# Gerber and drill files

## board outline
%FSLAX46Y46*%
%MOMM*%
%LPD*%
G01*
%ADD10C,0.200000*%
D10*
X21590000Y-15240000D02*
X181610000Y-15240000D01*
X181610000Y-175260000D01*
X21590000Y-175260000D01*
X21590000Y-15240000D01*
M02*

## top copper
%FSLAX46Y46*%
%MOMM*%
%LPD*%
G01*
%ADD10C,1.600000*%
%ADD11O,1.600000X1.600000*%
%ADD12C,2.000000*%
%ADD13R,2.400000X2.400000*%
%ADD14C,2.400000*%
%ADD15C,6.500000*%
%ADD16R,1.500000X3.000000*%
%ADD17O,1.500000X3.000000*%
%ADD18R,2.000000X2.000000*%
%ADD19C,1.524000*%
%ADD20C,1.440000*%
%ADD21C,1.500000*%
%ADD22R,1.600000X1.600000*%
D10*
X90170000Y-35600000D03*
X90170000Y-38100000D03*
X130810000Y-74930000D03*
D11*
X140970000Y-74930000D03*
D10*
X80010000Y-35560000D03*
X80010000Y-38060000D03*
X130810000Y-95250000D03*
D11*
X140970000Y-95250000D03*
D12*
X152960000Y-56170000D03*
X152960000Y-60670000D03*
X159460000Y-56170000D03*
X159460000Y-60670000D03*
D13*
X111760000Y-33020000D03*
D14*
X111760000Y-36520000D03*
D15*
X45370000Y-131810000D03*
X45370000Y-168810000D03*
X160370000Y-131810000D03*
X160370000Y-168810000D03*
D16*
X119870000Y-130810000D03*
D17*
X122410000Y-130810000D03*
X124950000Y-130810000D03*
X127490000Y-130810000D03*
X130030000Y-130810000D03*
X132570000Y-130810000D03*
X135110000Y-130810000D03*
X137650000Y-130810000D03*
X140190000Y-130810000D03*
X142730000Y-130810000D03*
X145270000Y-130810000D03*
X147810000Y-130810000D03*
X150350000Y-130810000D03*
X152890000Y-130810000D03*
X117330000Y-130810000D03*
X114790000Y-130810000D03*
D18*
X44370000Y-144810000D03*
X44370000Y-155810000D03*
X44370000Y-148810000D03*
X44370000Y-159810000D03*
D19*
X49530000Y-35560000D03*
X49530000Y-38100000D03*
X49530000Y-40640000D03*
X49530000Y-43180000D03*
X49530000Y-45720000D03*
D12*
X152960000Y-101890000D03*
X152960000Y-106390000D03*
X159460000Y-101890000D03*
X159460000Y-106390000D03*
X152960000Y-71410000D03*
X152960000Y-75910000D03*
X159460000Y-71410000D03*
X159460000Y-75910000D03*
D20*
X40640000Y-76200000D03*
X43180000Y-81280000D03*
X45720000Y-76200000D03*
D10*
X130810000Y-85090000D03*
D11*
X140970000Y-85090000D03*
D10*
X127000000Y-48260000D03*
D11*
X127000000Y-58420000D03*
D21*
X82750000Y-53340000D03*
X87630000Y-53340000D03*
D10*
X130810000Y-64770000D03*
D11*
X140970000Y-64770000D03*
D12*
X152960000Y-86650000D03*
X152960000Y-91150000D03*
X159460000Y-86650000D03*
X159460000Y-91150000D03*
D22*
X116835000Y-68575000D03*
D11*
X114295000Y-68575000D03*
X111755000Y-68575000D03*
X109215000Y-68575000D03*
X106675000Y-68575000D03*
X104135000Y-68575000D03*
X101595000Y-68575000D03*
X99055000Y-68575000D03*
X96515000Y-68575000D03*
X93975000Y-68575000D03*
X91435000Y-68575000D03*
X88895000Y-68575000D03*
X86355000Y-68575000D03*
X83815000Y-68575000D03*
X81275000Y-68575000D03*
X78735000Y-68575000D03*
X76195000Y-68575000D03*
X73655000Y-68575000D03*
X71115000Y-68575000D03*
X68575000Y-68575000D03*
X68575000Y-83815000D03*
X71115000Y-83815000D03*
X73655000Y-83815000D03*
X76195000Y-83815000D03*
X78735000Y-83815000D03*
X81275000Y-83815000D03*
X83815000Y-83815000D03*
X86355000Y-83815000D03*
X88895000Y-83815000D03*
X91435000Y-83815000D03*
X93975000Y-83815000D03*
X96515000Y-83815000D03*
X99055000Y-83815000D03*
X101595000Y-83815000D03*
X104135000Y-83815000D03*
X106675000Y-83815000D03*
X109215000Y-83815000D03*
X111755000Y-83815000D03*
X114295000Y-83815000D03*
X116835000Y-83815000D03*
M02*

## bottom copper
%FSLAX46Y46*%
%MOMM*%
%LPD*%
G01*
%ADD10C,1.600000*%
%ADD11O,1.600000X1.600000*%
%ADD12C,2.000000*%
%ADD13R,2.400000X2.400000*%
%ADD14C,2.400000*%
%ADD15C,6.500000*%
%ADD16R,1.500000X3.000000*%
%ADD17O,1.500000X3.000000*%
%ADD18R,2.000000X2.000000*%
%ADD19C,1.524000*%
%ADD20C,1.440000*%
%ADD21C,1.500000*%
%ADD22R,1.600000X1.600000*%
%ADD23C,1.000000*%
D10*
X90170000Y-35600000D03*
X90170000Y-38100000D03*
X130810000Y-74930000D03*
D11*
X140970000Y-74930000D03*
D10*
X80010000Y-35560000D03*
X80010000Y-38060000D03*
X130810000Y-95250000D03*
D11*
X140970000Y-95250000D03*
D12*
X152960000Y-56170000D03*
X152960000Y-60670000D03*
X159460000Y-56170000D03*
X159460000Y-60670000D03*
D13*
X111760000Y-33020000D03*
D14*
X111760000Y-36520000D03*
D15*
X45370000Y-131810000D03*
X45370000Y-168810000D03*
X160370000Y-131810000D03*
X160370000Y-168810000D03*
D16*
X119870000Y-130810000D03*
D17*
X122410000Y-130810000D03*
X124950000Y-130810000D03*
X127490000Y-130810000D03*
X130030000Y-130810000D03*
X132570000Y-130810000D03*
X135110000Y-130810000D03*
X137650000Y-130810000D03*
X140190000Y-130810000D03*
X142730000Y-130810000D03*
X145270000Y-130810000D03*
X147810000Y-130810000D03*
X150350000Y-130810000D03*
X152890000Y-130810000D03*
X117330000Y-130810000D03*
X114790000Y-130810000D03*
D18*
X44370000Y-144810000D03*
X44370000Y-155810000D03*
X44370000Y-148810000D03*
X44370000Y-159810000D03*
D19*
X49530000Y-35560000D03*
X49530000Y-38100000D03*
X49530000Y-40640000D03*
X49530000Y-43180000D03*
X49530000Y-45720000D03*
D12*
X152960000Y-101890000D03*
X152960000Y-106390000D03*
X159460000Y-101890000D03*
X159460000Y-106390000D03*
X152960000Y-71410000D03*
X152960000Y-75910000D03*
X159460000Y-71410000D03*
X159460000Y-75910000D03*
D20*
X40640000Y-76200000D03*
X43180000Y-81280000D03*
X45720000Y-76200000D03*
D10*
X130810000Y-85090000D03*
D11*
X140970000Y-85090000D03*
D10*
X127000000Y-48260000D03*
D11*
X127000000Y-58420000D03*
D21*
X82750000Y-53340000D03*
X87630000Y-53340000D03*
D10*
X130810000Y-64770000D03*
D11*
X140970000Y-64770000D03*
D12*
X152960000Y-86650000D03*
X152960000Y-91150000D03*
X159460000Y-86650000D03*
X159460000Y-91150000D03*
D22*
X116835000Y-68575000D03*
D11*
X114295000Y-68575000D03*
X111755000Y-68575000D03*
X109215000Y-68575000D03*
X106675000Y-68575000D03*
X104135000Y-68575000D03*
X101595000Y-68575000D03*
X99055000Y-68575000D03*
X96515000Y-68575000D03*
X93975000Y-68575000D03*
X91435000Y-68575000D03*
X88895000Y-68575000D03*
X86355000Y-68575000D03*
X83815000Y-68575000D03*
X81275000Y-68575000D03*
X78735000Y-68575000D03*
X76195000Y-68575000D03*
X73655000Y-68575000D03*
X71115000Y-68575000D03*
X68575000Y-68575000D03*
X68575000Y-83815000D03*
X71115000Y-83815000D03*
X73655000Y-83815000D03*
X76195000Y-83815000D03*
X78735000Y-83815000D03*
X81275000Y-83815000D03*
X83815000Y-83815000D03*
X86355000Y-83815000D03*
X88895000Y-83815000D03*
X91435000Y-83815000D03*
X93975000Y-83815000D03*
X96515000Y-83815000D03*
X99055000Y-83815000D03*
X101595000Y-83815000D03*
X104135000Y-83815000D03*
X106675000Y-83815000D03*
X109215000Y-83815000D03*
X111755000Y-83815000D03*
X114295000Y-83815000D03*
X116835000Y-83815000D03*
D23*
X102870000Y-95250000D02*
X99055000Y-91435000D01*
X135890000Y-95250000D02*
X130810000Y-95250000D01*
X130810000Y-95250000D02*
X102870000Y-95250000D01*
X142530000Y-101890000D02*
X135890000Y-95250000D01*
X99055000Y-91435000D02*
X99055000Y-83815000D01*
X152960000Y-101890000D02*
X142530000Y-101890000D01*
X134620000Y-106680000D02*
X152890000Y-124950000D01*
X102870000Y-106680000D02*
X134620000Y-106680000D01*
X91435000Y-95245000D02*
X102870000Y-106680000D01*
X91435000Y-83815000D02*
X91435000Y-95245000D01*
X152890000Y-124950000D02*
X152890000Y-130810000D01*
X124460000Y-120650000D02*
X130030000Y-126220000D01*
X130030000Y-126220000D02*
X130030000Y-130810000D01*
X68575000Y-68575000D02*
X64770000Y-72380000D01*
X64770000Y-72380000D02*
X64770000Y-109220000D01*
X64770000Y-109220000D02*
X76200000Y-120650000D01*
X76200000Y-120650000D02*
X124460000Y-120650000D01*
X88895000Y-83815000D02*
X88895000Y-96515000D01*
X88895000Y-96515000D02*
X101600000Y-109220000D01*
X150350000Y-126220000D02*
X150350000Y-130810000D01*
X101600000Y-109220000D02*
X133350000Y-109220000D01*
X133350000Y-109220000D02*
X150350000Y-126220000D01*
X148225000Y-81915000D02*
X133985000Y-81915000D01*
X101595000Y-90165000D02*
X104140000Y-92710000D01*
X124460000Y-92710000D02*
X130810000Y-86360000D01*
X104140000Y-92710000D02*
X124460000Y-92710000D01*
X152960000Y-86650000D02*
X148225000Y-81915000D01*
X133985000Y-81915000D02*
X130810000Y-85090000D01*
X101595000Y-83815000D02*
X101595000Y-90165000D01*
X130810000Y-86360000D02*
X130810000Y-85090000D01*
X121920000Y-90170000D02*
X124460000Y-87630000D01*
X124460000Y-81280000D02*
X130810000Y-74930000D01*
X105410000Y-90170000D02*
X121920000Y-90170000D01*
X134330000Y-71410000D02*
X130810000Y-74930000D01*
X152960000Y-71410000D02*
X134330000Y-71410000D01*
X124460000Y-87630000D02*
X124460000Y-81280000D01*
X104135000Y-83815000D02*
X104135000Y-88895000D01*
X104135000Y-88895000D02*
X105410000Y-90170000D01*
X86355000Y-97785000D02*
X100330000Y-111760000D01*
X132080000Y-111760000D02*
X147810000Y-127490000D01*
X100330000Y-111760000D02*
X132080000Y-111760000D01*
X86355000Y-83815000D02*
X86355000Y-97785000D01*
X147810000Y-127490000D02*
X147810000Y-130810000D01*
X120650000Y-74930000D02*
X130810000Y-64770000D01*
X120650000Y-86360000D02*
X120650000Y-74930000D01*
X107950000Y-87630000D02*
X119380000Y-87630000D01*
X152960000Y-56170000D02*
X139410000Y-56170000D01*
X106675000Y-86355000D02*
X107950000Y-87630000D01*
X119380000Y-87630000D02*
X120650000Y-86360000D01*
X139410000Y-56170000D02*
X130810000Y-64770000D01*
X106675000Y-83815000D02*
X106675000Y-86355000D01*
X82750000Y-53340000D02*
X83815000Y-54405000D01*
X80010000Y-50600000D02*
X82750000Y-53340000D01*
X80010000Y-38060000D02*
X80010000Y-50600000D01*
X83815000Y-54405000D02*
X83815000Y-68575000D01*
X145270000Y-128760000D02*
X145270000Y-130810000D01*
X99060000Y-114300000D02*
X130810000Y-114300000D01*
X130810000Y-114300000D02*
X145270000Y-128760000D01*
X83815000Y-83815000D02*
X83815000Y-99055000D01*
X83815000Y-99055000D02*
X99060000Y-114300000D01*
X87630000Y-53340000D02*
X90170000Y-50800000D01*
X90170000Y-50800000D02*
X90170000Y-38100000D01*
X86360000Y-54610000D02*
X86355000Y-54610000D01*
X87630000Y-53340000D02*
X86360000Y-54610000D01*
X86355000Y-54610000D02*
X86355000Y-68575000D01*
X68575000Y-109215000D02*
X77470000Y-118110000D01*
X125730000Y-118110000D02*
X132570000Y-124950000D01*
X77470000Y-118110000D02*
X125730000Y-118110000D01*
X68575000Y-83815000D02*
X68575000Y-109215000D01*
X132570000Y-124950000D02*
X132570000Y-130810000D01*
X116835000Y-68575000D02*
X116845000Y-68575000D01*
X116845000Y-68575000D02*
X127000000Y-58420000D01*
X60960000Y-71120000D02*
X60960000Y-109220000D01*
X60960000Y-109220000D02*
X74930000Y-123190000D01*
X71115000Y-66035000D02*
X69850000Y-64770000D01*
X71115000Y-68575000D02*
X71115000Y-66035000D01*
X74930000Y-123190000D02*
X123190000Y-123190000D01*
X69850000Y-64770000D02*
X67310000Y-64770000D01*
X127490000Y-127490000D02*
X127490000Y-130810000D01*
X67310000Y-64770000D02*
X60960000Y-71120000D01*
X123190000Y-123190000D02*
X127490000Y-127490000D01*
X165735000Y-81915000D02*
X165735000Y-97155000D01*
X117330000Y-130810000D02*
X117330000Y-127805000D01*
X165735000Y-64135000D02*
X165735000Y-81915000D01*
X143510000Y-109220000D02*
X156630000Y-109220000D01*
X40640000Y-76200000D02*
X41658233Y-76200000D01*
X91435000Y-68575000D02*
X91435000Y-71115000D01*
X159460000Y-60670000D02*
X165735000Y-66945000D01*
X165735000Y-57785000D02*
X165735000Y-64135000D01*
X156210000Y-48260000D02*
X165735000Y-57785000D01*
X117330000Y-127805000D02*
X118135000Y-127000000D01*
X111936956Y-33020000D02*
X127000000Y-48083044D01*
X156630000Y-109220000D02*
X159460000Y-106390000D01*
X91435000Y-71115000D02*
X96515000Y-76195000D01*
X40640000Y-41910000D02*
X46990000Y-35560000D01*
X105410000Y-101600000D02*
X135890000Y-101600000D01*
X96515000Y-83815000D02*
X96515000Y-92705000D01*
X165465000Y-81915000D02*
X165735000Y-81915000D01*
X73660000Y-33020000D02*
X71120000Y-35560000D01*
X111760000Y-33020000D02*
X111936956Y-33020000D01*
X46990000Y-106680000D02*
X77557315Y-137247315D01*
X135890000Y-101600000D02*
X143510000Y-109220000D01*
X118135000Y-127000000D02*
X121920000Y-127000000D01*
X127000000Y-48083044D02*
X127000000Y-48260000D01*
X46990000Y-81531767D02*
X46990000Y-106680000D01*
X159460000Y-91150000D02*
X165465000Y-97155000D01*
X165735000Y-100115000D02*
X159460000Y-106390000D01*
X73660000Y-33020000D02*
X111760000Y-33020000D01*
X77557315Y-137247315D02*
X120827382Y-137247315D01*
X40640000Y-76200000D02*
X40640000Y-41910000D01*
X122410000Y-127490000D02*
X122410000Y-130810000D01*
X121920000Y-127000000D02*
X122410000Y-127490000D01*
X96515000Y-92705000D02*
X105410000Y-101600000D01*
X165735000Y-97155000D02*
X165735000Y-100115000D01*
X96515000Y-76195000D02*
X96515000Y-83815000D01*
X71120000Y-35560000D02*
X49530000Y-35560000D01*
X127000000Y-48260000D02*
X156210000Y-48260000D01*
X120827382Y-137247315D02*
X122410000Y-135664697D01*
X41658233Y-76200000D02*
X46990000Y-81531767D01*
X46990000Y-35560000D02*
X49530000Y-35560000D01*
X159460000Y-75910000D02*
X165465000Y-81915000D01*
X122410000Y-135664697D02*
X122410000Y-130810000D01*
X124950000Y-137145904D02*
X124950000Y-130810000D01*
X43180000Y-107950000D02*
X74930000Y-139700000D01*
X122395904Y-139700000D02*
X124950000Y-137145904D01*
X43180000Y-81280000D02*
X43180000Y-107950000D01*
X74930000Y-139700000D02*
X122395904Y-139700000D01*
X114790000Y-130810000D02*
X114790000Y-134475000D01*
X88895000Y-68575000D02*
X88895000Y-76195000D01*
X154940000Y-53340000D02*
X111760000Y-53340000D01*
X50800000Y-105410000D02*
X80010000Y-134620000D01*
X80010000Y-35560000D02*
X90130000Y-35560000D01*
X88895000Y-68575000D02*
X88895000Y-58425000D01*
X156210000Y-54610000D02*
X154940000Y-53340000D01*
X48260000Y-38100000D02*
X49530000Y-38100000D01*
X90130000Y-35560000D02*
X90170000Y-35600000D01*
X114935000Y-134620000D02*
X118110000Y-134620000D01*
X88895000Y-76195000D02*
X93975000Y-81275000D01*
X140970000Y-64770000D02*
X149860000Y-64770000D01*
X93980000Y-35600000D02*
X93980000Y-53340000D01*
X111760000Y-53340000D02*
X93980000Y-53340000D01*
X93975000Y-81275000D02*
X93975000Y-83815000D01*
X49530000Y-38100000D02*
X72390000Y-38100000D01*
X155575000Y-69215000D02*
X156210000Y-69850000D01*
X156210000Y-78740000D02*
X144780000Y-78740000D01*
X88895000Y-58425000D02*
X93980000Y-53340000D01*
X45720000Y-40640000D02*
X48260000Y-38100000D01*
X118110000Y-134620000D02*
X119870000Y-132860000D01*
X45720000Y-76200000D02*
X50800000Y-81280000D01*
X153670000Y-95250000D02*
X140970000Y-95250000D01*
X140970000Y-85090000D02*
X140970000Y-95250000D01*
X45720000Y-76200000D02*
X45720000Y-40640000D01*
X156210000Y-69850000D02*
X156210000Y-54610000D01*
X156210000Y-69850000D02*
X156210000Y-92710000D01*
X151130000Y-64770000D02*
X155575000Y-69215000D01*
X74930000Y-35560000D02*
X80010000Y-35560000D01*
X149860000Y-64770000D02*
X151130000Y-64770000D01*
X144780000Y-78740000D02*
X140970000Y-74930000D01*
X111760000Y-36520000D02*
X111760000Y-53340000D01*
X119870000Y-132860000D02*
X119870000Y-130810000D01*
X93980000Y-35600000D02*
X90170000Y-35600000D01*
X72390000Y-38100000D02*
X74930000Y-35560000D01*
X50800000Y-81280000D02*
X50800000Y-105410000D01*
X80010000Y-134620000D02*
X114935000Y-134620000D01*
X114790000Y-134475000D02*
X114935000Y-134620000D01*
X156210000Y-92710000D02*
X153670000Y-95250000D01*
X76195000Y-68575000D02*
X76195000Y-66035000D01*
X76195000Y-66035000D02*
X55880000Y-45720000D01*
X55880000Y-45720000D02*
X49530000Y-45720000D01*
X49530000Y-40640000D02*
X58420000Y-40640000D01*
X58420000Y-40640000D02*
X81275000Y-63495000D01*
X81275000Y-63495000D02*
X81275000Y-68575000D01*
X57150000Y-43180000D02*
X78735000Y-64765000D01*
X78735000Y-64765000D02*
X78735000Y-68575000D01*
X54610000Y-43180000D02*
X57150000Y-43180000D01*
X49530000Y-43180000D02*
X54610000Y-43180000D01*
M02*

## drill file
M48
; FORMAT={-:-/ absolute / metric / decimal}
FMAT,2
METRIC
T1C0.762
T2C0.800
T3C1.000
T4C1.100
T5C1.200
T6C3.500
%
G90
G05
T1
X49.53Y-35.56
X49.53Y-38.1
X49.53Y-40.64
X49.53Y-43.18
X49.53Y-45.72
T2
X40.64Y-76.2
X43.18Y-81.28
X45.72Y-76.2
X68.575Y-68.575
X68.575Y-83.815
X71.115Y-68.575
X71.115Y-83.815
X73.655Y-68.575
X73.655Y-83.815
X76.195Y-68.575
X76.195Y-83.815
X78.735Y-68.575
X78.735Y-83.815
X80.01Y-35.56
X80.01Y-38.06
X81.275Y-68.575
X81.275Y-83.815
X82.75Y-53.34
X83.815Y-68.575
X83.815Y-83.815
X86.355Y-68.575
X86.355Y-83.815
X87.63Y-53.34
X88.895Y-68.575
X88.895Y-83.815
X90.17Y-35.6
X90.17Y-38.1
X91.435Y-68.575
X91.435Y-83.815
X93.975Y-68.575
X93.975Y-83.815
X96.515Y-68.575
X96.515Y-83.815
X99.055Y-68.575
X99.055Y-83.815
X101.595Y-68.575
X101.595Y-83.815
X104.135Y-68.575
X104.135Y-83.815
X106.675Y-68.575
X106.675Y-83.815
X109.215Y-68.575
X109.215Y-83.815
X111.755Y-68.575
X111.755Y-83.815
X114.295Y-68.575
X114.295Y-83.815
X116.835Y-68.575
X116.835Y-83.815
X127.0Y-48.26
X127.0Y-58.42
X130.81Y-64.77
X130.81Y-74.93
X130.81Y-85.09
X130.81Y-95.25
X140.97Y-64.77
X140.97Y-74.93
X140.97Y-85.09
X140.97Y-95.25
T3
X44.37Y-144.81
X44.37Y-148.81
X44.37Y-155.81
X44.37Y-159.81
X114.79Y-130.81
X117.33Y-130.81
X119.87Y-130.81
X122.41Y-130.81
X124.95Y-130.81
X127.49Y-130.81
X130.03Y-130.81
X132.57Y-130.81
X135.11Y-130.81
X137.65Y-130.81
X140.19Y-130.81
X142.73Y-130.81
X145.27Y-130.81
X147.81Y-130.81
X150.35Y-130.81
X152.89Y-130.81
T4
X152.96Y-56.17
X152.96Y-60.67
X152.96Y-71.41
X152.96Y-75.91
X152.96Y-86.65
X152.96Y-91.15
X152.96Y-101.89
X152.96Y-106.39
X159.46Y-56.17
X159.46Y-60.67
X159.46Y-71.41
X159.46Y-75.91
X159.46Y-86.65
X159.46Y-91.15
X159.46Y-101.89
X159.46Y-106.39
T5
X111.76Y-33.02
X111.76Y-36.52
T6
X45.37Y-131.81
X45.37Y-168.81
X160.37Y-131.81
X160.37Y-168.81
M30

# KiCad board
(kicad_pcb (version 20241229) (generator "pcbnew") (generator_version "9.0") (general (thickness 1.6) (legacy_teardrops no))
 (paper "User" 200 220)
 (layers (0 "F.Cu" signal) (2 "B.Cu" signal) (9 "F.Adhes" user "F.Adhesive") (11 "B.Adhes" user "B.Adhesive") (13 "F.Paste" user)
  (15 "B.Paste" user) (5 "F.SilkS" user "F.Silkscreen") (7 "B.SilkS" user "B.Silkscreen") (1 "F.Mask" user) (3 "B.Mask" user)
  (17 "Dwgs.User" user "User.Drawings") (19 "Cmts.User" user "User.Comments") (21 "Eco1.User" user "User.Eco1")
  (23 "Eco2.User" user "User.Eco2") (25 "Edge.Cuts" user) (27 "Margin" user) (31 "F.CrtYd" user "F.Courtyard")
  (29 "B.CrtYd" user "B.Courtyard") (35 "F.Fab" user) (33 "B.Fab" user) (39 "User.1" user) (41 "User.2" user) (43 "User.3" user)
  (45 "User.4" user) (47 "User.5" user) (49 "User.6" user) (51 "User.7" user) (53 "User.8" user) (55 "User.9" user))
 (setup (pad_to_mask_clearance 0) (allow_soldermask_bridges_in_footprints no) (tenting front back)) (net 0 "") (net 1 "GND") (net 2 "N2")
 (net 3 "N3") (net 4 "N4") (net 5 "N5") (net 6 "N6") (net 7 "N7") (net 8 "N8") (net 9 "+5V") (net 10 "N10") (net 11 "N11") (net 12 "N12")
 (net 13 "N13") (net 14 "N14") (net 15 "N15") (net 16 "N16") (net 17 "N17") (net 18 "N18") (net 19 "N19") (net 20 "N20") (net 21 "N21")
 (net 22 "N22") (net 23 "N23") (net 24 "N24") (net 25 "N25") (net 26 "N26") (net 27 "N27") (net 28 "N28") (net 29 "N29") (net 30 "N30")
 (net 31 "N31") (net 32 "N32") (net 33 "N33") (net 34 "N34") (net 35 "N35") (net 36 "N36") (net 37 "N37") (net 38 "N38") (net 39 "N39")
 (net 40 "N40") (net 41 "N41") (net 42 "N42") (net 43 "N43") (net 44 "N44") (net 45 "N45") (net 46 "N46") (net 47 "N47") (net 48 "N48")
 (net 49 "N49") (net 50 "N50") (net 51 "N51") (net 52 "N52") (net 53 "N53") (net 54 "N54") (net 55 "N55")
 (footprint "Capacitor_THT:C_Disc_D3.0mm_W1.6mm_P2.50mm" (layer "F.Cu") (at 90.17 35.6 -90)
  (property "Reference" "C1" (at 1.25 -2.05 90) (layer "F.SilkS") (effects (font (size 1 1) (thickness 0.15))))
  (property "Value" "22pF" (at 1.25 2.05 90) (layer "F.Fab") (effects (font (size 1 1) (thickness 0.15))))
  (pad "1" thru_hole circle (at 0 0 270) (size 1.6 1.6) (drill 0.8) (layers "*.Cu" "*.Mask") (remove_unused_layers no) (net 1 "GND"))
  (pad "2" thru_hole circle (at 2.5 0 270) (size 1.6 1.6) (drill 0.8) (layers "*.Cu" "*.Mask") (remove_unused_layers no) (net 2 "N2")))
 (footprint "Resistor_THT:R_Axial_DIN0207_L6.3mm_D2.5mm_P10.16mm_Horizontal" (layer "F.Cu") (at 130.81 74.93)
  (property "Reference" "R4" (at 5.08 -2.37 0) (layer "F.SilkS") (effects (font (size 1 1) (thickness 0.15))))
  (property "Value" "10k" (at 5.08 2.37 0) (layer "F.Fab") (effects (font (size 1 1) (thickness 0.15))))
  (pad "1" thru_hole circle (at 0 0) (size 1.6 1.6) (drill 0.8) (layers "*.Cu" "*.Mask") (remove_unused_layers no) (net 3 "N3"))
  (pad "2" thru_hole oval (at 10.16 0) (size 1.6 1.6) (drill 0.8) (layers "*.Cu" "*.Mask") (remove_unused_layers no) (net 1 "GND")))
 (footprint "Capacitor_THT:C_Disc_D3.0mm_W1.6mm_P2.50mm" (layer "F.Cu") (at 80.01 35.56 -90)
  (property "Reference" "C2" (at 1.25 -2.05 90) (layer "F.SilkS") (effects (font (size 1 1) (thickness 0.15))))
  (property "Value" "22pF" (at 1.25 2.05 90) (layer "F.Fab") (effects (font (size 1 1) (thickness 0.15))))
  (pad "1" thru_hole circle (at 0 0 270) (size 1.6 1.6) (drill 0.8) (layers "*.Cu" "*.Mask") (remove_unused_layers no) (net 1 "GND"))
  (pad "2" thru_hole circle (at 2.5 0 270) (size 1.6 1.6) (drill 0.8) (layers "*.Cu" "*.Mask") (remove_unused_layers no) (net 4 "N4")))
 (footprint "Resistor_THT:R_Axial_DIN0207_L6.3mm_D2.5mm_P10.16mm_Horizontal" (layer "F.Cu") (at 130.81 95.25)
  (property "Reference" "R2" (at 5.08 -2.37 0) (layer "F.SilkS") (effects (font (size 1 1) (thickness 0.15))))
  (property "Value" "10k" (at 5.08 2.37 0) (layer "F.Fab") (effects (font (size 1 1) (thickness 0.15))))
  (pad "1" thru_hole circle (at 0 0) (size 1.6 1.6) (drill 0.8) (layers "*.Cu" "*.Mask") (remove_unused_layers no) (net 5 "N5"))
  (pad "2" thru_hole oval (at 10.16 0) (size 1.6 1.6) (drill 0.8) (layers "*.Cu" "*.Mask") (remove_unused_layers no) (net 1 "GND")))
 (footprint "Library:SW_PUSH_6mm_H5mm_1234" (layer "F.Cu") (at 152.96 56.17)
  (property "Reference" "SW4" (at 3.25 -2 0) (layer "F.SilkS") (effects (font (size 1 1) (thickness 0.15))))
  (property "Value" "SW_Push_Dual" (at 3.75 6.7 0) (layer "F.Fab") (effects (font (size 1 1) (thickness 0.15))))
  (pad "1" thru_hole circle (at 0 0 90) (size 2 2) (drill 1.1) (layers "*.Cu" "*.Mask") (remove_unused_layers no) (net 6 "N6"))
  (pad "2" thru_hole circle (at 0 4.5 90) (size 2 2) (drill 1.1) (layers "*.Cu" "*.Mask") (remove_unused_layers no) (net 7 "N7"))
  (pad "3" thru_hole circle (at 6.5 0 90) (size 2 2) (drill 1.1) (layers "*.Cu" "*.Mask") (remove_unused_layers no) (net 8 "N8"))
  (pad "4" thru_hole circle (at 6.5 4.5 90) (size 2 2) (drill 1.1) (layers "*.Cu" "*.Mask") (remove_unused_layers no) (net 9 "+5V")))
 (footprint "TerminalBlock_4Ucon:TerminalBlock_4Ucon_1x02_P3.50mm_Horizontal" (layer "F.Cu") (at 111.76 33.02 -90)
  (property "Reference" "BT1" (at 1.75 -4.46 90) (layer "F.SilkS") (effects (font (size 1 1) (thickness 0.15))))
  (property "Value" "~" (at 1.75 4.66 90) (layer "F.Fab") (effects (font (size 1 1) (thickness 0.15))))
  (pad "1" thru_hole rect (at 0 0 270) (size 2.4 2.4) (drill 1.2) (layers "*.Cu" "*.Mask") (remove_unused_layers no) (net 9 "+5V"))
  (pad "2" thru_hole circle (at 3.5 0 270) (size 2.4 2.4) (drill 1.2) (layers "*.Cu" "*.Mask") (remove_unused_layers no) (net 1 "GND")))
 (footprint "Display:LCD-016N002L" (layer "F.Cu") (at 119.87 130.81)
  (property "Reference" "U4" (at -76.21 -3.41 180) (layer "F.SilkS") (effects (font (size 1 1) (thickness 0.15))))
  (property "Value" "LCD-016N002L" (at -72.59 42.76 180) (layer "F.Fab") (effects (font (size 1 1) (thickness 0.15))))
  (pad "" thru_hole circle (at -74.5 1 180) (size 6.5 6.5) (drill 3.5) (layers "*.Cu" "*.Mask") (remove_unused_layers no))
  (pad "" thru_hole circle (at -74.5 38 180) (size 6.5 6.5) (drill 3.5) (layers "*.Cu" "*.Mask") (remove_unused_layers no))
  (pad "" thru_hole circle (at 40.5 1 180) (size 6.5 6.5) (drill 3.5) (layers "*.Cu" "*.Mask") (remove_unused_layers no))
  (pad "" thru_hole circle (at 40.5 38 180) (size 6.5 6.5) (drill 3.5) (layers "*.Cu" "*.Mask") (remove_unused_layers no))
  (pad "1" thru_hole rect (at 0 0 180) (size 1.5 3) (drill 1) (layers "*.Cu" "*.Mask") (remove_unused_layers no) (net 1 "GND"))
  (pad "2" thru_hole oval (at 2.54 0 180) (size 1.5 3) (drill 1) (layers "*.Cu" "*.Mask") (remove_unused_layers no) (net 9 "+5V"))
  (pad "3" thru_hole oval (at 5.08 0 180) (size 1.5 3) (drill 1) (layers "*.Cu" "*.Mask") (remove_unused_layers no) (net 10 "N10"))
  (pad "4" thru_hole oval (at 7.62 0 180) (size 1.5 3) (drill 1) (layers "*.Cu" "*.Mask") (remove_unused_layers no) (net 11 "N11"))
  (pad "5" thru_hole oval (at 10.16 0 180) (size 1.5 3) (drill 1) (layers "*.Cu" "*.Mask") (remove_unused_layers no) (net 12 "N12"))
  (pad "6" thru_hole oval (at 12.7 0 180) (size 1.5 3) (drill 1) (layers "*.Cu" "*.Mask") (remove_unused_layers no) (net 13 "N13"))
  (pad "7" thru_hole oval (at 15.24 0 180) (size 1.5 3) (drill 1) (layers "*.Cu" "*.Mask") (remove_unused_layers no) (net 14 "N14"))
  (pad "8" thru_hole oval (at 17.78 0 180) (size 1.5 3) (drill 1) (layers "*.Cu" "*.Mask") (remove_unused_layers no) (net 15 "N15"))
  (pad "9" thru_hole oval (at 20.32 0 180) (size 1.5 3) (drill 1) (layers "*.Cu" "*.Mask") (remove_unused_layers no) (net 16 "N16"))
  (pad "10" thru_hole oval (at 22.86 0 180) (size 1.5 3) (drill 1) (layers "*.Cu" "*.Mask") (remove_unused_layers no) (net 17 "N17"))
  (pad "11" thru_hole oval (at 25.4 0 180) (size 1.5 3) (drill 1) (layers "*.Cu" "*.Mask") (remove_unused_layers no) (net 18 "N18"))
  (pad "12" thru_hole oval (at 27.94 0 180) (size 1.5 3) (drill 1) (layers "*.Cu" "*.Mask") (remove_unused_layers no) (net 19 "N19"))
  (pad "13" thru_hole oval (at 30.48 0 180) (size 1.5 3) (drill 1) (layers "*.Cu" "*.Mask") (remove_unused_layers no) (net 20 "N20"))
  (pad "14" thru_hole oval (at 33.02 0 180) (size 1.5 3) (drill 1) (layers "*.Cu" "*.Mask") (remove_unused_layers no) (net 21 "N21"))
  (pad "15" thru_hole oval (at -2.54 0 180) (size 1.5 3) (drill 1) (layers "*.Cu" "*.Mask") (remove_unused_layers no) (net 9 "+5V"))
  (pad "16" thru_hole oval (at -5.08 0 180) (size 1.5 3) (drill 1) (layers "*.Cu" "*.Mask") (remove_unused_layers no) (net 1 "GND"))
  (pad "A1" thru_hole rect (at -75.5 14 180) (size 2 2) (drill 1) (layers "*.Cu" "*.Mask") (remove_unused_layers no) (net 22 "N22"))
  (pad "A2" thru_hole rect (at -75.5 25 180) (size 2 2) (drill 1) (layers "*.Cu" "*.Mask") (remove_unused_layers no) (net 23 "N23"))
  (pad "K1" thru_hole rect (at -75.5 18 180) (size 2 2) (drill 1) (layers "*.Cu" "*.Mask") (remove_unused_layers no) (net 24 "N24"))
  (pad "K2" thru_hole rect (at -75.5 29 180) (size 2 2) (drill 1) (layers "*.Cu" "*.Mask") (remove_unused_layers no) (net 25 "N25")))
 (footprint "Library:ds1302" (layer "F.Cu") (at 49.53 40.64 -90)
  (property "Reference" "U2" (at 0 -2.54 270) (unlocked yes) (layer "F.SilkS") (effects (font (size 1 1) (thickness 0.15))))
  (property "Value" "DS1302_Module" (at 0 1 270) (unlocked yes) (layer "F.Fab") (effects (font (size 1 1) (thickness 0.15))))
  (pad "1" thru_hole circle (at -5.08 0 270) (size 1.524 1.524) (drill 0.762) (layers "*.Cu" "*.Mask") (remove_unused_layers no)
   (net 9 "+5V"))
  (pad "2" thru_hole circle (at -2.54 0 270) (size 1.524 1.524) (drill 0.762) (layers "*.Cu" "*.Mask") (remove_unused_layers no)
   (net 1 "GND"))
  (pad "3" thru_hole circle (at 0 0 270) (size 1.524 1.524) (drill 0.762) (layers "*.Cu" "*.Mask") (remove_unused_layers no) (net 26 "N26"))
  (pad "4" thru_hole circle (at 2.54 0 270) (size 1.524 1.524) (drill 0.762) (layers "*.Cu" "*.Mask") (remove_unused_layers no)
   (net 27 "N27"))
  (pad "5" thru_hole circle (at 5.08 0 270) (size 1.524 1.524) (drill 0.762) (layers "*.Cu" "*.Mask") (remove_unused_layers no)
   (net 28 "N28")))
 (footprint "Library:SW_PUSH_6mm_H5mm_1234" (layer "F.Cu") (at 152.96 101.89)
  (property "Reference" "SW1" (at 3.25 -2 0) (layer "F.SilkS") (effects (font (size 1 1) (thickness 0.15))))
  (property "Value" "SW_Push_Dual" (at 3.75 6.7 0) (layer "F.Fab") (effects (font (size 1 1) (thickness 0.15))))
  (pad "1" thru_hole circle (at 0 0 90) (size 2 2) (drill 1.1) (layers "*.Cu" "*.Mask") (remove_unused_layers no) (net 5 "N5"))
  (pad "2" thru_hole circle (at 0 4.5 90) (size 2 2) (drill 1.1) (layers "*.Cu" "*.Mask") (remove_unused_layers no) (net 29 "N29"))
  (pad "3" thru_hole circle (at 6.5 0 90) (size 2 2) (drill 1.1) (layers "*.Cu" "*.Mask") (remove_unused_layers no) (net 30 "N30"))
  (pad "4" thru_hole circle (at 6.5 4.5 90) (size 2 2) (drill 1.1) (layers "*.Cu" "*.Mask") (remove_unused_layers no) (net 9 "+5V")))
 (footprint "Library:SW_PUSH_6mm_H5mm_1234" (layer "F.Cu") (at 152.96 71.41)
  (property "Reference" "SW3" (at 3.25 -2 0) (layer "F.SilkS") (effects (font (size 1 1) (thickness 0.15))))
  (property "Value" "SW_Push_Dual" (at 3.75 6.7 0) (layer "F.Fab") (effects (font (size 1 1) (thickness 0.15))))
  (pad "1" thru_hole circle (at 0 0 90) (size 2 2) (drill 1.1) (layers "*.Cu" "*.Mask") (remove_unused_layers no) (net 3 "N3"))
  (pad "2" thru_hole circle (at 0 4.5 90) (size 2 2) (drill 1.1) (layers "*.Cu" "*.Mask") (remove_unused_layers no) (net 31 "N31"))
  (pad "3" thru_hole circle (at 6.5 0 90) (size 2 2) (drill 1.1) (layers "*.Cu" "*.Mask") (remove_unused_layers no) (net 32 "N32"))
  (pad "4" thru_hole circle (at 6.5 4.5 90) (size 2 2) (drill 1.1) (layers "*.Cu" "*.Mask") (remove_unused_layers no) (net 9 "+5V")))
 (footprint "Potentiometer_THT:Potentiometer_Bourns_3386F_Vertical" (layer "F.Cu") (at 40.64 76.2 -90)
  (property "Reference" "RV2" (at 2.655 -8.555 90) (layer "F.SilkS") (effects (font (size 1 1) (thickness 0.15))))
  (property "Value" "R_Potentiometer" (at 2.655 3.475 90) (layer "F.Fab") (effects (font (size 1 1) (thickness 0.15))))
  (pad "1" thru_hole circle (at 0 0 270) (size 1.44 1.44) (drill 0.8) (layers "*.Cu" "*.Mask") (remove_unused_layers no) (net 9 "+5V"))
  (pad "2" thru_hole circle (at 5.08 -2.54 270) (size 1.44 1.44) (drill 0.8) (layers "*.Cu" "*.Mask") (remove_unused_layers no)
   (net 10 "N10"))
  (pad "3" thru_hole circle (at 0 -5.08 270) (size 1.44 1.44) (drill 0.8) (layers "*.Cu" "*.Mask") (remove_unused_layers no) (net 1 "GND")))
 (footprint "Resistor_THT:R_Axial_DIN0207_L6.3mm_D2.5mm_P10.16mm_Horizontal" (layer "F.Cu") (at 130.81 85.09)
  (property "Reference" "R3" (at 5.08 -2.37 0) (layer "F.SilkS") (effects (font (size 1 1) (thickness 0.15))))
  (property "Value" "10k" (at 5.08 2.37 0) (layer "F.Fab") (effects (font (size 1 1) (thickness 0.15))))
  (pad "1" thru_hole circle (at 0 0) (size 1.6 1.6) (drill 0.8) (layers "*.Cu" "*.Mask") (remove_unused_layers no) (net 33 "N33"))
  (pad "2" thru_hole oval (at 10.16 0) (size 1.6 1.6) (drill 0.8) (layers "*.Cu" "*.Mask") (remove_unused_layers no) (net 1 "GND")))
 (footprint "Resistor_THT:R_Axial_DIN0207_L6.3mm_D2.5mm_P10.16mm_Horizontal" (layer "F.Cu") (at 127 48.26 -90)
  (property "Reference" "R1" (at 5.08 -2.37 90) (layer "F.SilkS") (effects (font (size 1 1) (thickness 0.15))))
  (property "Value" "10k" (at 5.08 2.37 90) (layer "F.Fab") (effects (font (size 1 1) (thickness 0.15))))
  (pad "1" thru_hole circle (at 0 0 270) (size 1.6 1.6) (drill 0.8) (layers "*.Cu" "*.Mask") (remove_unused_layers no) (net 9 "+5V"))
  (pad "2" thru_hole oval (at 10.16 0 270) (size 1.6 1.6) (drill 0.8) (layers "*.Cu" "*.Mask") (remove_unused_layers no) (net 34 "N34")))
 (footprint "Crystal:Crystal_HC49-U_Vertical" (layer "F.Cu") (at 82.75 53.34)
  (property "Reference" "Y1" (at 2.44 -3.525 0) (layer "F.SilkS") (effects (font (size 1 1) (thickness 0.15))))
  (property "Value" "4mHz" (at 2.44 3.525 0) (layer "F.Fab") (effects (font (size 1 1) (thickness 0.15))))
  (pad "1" thru_hole circle (at 0 0) (size 1.5 1.5) (drill 0.8) (layers "*.Cu" "*.Mask") (remove_unused_layers no) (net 4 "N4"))
  (pad "2" thru_hole circle (at 4.88 0) (size 1.5 1.5) (drill 0.8) (layers "*.Cu" "*.Mask") (remove_unused_layers no) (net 2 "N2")))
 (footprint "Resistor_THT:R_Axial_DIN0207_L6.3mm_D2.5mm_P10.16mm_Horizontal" (layer "F.Cu") (at 130.81 64.77)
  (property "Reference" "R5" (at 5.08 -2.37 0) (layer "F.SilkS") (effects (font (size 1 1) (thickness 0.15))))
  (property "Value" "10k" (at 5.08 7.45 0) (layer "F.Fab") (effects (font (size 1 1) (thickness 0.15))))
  (pad "1" thru_hole circle (at 0 0) (size 1.6 1.6) (drill 0.8) (layers "*.Cu" "*.Mask") (remove_unused_layers no) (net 6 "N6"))
  (pad "2" thru_hole oval (at 10.16 0) (size 1.6 1.6) (drill 0.8) (layers "*.Cu" "*.Mask") (remove_unused_layers no) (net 1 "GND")))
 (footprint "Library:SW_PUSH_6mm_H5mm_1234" (layer "F.Cu") (at 152.96 86.65)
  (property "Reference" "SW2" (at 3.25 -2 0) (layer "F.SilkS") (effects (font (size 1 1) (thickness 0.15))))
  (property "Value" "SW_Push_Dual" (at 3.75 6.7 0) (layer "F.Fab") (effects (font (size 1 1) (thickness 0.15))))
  (pad "1" thru_hole circle (at 0 0 90) (size 2 2) (drill 1.1) (layers "*.Cu" "*.Mask") (remove_unused_layers no) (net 33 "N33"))
  (pad "2" thru_hole circle (at 0 4.5 90) (size 2 2) (drill 1.1) (layers "*.Cu" "*.Mask") (remove_unused_layers no) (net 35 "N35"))
  (pad "3" thru_hole circle (at 6.5 0 90) (size 2 2) (drill 1.1) (layers "*.Cu" "*.Mask") (remove_unused_layers no) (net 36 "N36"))
  (pad "4" thru_hole circle (at 6.5 4.5 90) (size 2 2) (drill 1.1) (layers "*.Cu" "*.Mask") (remove_unused_layers no) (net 9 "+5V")))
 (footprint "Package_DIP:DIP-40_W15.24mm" (layer "F.Cu") (at 116.835 68.575 -90)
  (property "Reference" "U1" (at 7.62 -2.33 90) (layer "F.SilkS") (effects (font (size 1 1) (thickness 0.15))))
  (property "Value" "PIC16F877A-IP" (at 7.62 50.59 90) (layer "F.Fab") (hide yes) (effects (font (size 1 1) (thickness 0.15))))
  (pad "1" thru_hole rect (at 0 0 270) (size 1.6 1.6) (drill 0.8) (layers "*.Cu" "*.Mask") (remove_unused_layers no) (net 34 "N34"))
  (pad "2" thru_hole oval (at 0 2.54 270) (size 1.6 1.6) (drill 0.8) (layers "*.Cu" "*.Mask") (remove_unused_layers no) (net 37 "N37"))
  (pad "3" thru_hole oval (at 0 5.08 270) (size 1.6 1.6) (drill 0.8) (layers "*.Cu" "*.Mask") (remove_unused_layers no) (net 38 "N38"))
  (pad "4" thru_hole oval (at 0 7.62 270) (size 1.6 1.6) (drill 0.8) (layers "*.Cu" "*.Mask") (remove_unused_layers no) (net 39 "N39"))
  (pad "5" thru_hole oval (at 0 10.16 270) (size 1.6 1.6) (drill 0.8) (layers "*.Cu" "*.Mask") (remove_unused_layers no) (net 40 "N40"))
  (pad "6" thru_hole oval (at 0 12.7 270) (size 1.6 1.6) (drill 0.8) (layers "*.Cu" "*.Mask") (remove_unused_layers no) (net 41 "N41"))
  (pad "7" thru_hole oval (at 0 15.24 270) (size 1.6 1.6) (drill 0.8) (layers "*.Cu" "*.Mask") (remove_unused_layers no) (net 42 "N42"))
  (pad "8" thru_hole oval (at 0 17.78 270) (size 1.6 1.6) (drill 0.8) (layers "*.Cu" "*.Mask") (remove_unused_layers no) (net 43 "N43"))
  (pad "9" thru_hole oval (at 0 20.32 270) (size 1.6 1.6) (drill 0.8) (layers "*.Cu" "*.Mask") (remove_unused_layers no) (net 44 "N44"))
  (pad "10" thru_hole oval (at 0 22.86 270) (size 1.6 1.6) (drill 0.8) (layers "*.Cu" "*.Mask") (remove_unused_layers no) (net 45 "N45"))
  (pad "11" thru_hole oval (at 0 25.4 270) (size 1.6 1.6) (drill 0.8) (layers "*.Cu" "*.Mask") (remove_unused_layers no) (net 9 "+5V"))
  (pad "12" thru_hole oval (at 0 27.94 270) (size 1.6 1.6) (drill 0.8) (layers "*.Cu" "*.Mask") (remove_unused_layers no) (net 1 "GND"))
  (pad "13" thru_hole oval (at 0 30.48 270) (size 1.6 1.6) (drill 0.8) (layers "*.Cu" "*.Mask") (remove_unused_layers no) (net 2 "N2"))
  (pad "14" thru_hole oval (at 0 33.02 270) (size 1.6 1.6) (drill 0.8) (layers "*.Cu" "*.Mask") (remove_unused_layers no) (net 4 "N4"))
  (pad "15" thru_hole oval (at 0 35.56 270) (size 1.6 1.6) (drill 0.8) (layers "*.Cu" "*.Mask") (remove_unused_layers no) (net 26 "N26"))
  (pad "16" thru_hole oval (at 0 38.1 270) (size 1.6 1.6) (drill 0.8) (layers "*.Cu" "*.Mask") (remove_unused_layers no) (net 27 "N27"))
  (pad "17" thru_hole oval (at 0 40.64 270) (size 1.6 1.6) (drill 0.8) (layers "*.Cu" "*.Mask") (remove_unused_layers no) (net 28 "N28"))
  (pad "18" thru_hole oval (at 0 43.18 270) (size 1.6 1.6) (drill 0.8) (layers "*.Cu" "*.Mask") (remove_unused_layers no) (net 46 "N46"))
  (pad "19" thru_hole oval (at 0 45.72 270) (size 1.6 1.6) (drill 0.8) (layers "*.Cu" "*.Mask") (remove_unused_layers no) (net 11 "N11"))
  (pad "20" thru_hole oval (at 0 48.26 270) (size 1.6 1.6) (drill 0.8) (layers "*.Cu" "*.Mask") (remove_unused_layers no) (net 12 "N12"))
  (pad "21" thru_hole oval (at 15.24 48.26 270) (size 1.6 1.6) (drill 0.8) (layers "*.Cu" "*.Mask") (remove_unused_layers no) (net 13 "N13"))
  (pad "22" thru_hole oval (at 15.24 45.72 270) (size 1.6 1.6) (drill 0.8) (layers "*.Cu" "*.Mask") (remove_unused_layers no) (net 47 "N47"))
  (pad "23" thru_hole oval (at 15.24 43.18 270) (size 1.6 1.6) (drill 0.8) (layers "*.Cu" "*.Mask") (remove_unused_layers no) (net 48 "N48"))
  (pad "24" thru_hole oval (at 15.24 40.64 270) (size 1.6 1.6) (drill 0.8) (layers "*.Cu" "*.Mask") (remove_unused_layers no) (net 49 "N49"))
  (pad "25" thru_hole oval (at 15.24 38.1 270) (size 1.6 1.6) (drill 0.8) (layers "*.Cu" "*.Mask") (remove_unused_layers no) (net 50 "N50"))
  (pad "26" thru_hole oval (at 15.24 35.56 270) (size 1.6 1.6) (drill 0.8) (layers "*.Cu" "*.Mask") (remove_unused_layers no) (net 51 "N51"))
  (pad "27" thru_hole oval (at 15.24 33.02 270) (size 1.6 1.6) (drill 0.8) (layers "*.Cu" "*.Mask") (remove_unused_layers no) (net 18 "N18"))
  (pad "28" thru_hole oval (at 15.24 30.48 270) (size 1.6 1.6) (drill 0.8) (layers "*.Cu" "*.Mask") (remove_unused_layers no) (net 19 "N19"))
  (pad "29" thru_hole oval (at 15.24 27.94 270) (size 1.6 1.6) (drill 0.8) (layers "*.Cu" "*.Mask") (remove_unused_layers no) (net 20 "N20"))
  (pad "30" thru_hole oval (at 15.24 25.4 270) (size 1.6 1.6) (drill 0.8) (layers "*.Cu" "*.Mask") (remove_unused_layers no) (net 21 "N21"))
  (pad "31" thru_hole oval (at 15.24 22.86 270) (size 1.6 1.6) (drill 0.8) (layers "*.Cu" "*.Mask") (remove_unused_layers no) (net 1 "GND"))
  (pad "32" thru_hole oval (at 15.24 20.32 270) (size 1.6 1.6) (drill 0.8) (layers "*.Cu" "*.Mask") (remove_unused_layers no) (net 9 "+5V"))
  (pad "33" thru_hole oval (at 15.24 17.78 270) (size 1.6 1.6) (drill 0.8) (layers "*.Cu" "*.Mask") (remove_unused_layers no) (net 5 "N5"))
  (pad "34" thru_hole oval (at 15.24 15.24 270) (size 1.6 1.6) (drill 0.8) (layers "*.Cu" "*.Mask") (remove_unused_layers no) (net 33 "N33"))
  (pad "35" thru_hole oval (at 15.24 12.7 270) (size 1.6 1.6) (drill 0.8) (layers "*.Cu" "*.Mask") (remove_unused_layers no) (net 3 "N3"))
  (pad "36" thru_hole oval (at 15.24 10.16 270) (size 1.6 1.6) (drill 0.8) (layers "*.Cu" "*.Mask") (remove_unused_layers no) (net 6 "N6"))
  (pad "37" thru_hole oval (at 15.24 7.62 270) (size 1.6 1.6) (drill 0.8) (layers "*.Cu" "*.Mask") (remove_unused_layers no) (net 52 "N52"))
  (pad "38" thru_hole oval (at 15.24 5.08 270) (size 1.6 1.6) (drill 0.8) (layers "*.Cu" "*.Mask") (remove_unused_layers no) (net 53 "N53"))
  (pad "39" thru_hole oval (at 15.24 2.54 270) (size 1.6 1.6) (drill 0.8) (layers "*.Cu" "*.Mask") (remove_unused_layers no) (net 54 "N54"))
  (pad "40" thru_hole oval (at 15.24 0 270) (size 1.6 1.6) (drill 0.8) (layers "*.Cu" "*.Mask") (remove_unused_layers no) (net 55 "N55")))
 (gr_rect (start 21.59 15.24) (end 181.61 175.26) (stroke (width 0.2) (type default)) (fill no) (layer "Edge.Cuts"))
 (segment (start 102.87 95.25) (end 99.055 91.435) (width 1) (layer "B.Cu") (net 5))
 (segment (start 135.89 95.25) (end 130.81 95.25) (width 1) (layer "B.Cu") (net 5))
 (segment (start 130.81 95.25) (end 102.87 95.25) (width 1) (layer "B.Cu") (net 5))
 (segment (start 142.53 101.89) (end 135.89 95.25) (width 1) (layer "B.Cu") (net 5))
 (segment (start 99.055 91.435) (end 99.055 83.815) (width 1) (layer "B.Cu") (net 5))
 (segment (start 152.96 101.89) (end 142.53 101.89) (width 1) (layer "B.Cu") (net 5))
 (segment (start 134.62 106.68) (end 152.89 124.95) (width 1) (layer "B.Cu") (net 21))
 (segment (start 102.87 106.68) (end 134.62 106.68) (width 1) (layer "B.Cu") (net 21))
 (segment (start 91.435 95.245) (end 102.87 106.68) (width 1) (layer "B.Cu") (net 21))
 (segment (start 91.435 83.815) (end 91.435 95.245) (width 1) (layer "B.Cu") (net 21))
 (segment (start 152.89 124.95) (end 152.89 130.81) (width 1) (layer "B.Cu") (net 21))
 (segment (start 124.46 120.65) (end 130.03 126.22) (width 1) (layer "B.Cu") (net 12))
 (segment (start 130.03 126.22) (end 130.03 130.81) (width 1) (layer "B.Cu") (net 12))
 (segment (start 68.575 68.575) (end 64.77 72.38) (width 1) (layer "B.Cu") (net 12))
 (segment (start 64.77 72.38) (end 64.77 109.22) (width 1) (layer "B.Cu") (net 12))
 (segment (start 64.77 109.22) (end 76.2 120.65) (width 1) (layer "B.Cu") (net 12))
 (segment (start 76.2 120.65) (end 124.46 120.65) (width 1) (layer "B.Cu") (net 12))
 (segment (start 88.895 83.815) (end 88.895 96.515) (width 1) (layer "B.Cu") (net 20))
 (segment (start 88.895 96.515) (end 101.6 109.22) (width 1) (layer "B.Cu") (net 20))
 (segment (start 150.35 126.22) (end 150.35 130.81) (width 1) (layer "B.Cu") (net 20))
 (segment (start 101.6 109.22) (end 133.35 109.22) (width 1) (layer "B.Cu") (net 20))
 (segment (start 133.35 109.22) (end 150.35 126.22) (width 1) (layer "B.Cu") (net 20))
 (segment (start 148.225 81.915) (end 133.985 81.915) (width 1) (layer "B.Cu") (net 33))
 (segment (start 101.595 90.165) (end 104.14 92.71) (width 1) (layer "B.Cu") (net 33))
 (segment (start 124.46 92.71) (end 130.81 86.36) (width 1) (layer "B.Cu") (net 33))
 (segment (start 104.14 92.71) (end 124.46 92.71) (width 1) (layer "B.Cu") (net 33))
 (segment (start 152.96 86.65) (end 148.225 81.915) (width 1) (layer "B.Cu") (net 33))
 (segment (start 133.985 81.915) (end 130.81 85.09) (width 1) (layer "B.Cu") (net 33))
 (segment (start 101.595 83.815) (end 101.595 90.165) (width 1) (layer "B.Cu") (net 33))
 (segment (start 130.81 86.36) (end 130.81 85.09) (width 1) (layer "B.Cu") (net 33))
 (segment (start 121.92 90.17) (end 124.46 87.63) (width 1) (layer "B.Cu") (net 3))
 (segment (start 124.46 81.28) (end 130.81 74.93) (width 1) (layer "B.Cu") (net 3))
 (segment (start 105.41 90.17) (end 121.92 90.17) (width 1) (layer "B.Cu") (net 3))
 (segment (start 134.33 71.41) (end 130.81 74.93) (width 1) (layer "B.Cu") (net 3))
 (segment (start 152.96 71.41) (end 134.33 71.41) (width 1) (layer "B.Cu") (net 3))
 (segment (start 124.46 87.63) (end 124.46 81.28) (width 1) (layer "B.Cu") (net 3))
 (segment (start 104.135 83.815) (end 104.135 88.895) (width 1) (layer "B.Cu") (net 3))
 (segment (start 104.135 88.895) (end 105.41 90.17) (width 1) (layer "B.Cu") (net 3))
 (segment (start 86.355 97.785) (end 100.33 111.76) (width 1) (layer "B.Cu") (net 19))
 (segment (start 132.08 111.76) (end 147.81 127.49) (width 1) (layer "B.Cu") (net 19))
 (segment (start 100.33 111.76) (end 132.08 111.76) (width 1) (layer "B.Cu") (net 19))
 (segment (start 86.355 83.815) (end 86.355 97.785) (width 1) (layer "B.Cu") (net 19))
 (segment (start 147.81 127.49) (end 147.81 130.81) (width 1) (layer "B.Cu") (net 19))
 (segment (start 120.65 74.93) (end 130.81 64.77) (width 1) (layer "B.Cu") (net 6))
 (segment (start 120.65 86.36) (end 120.65 74.93) (width 1) (layer "B.Cu") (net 6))
 (segment (start 107.95 87.63) (end 119.38 87.63) (width 1) (layer "B.Cu") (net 6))
 (segment (start 152.96 56.17) (end 139.41 56.17) (width 1) (layer "B.Cu") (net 6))
 (segment (start 106.675 86.355) (end 107.95 87.63) (width 1) (layer "B.Cu") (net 6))
 (segment (start 119.38 87.63) (end 120.65 86.36) (width 1) (layer "B.Cu") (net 6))
 (segment (start 139.41 56.17) (end 130.81 64.77) (width 1) (layer "B.Cu") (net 6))
 (segment (start 106.675 83.815) (end 106.675 86.355) (width 1) (layer "B.Cu") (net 6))
 (segment (start 82.75 53.34) (end 83.815 54.405) (width 1) (layer "B.Cu") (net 4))
 (segment (start 80.01 50.6) (end 82.75 53.34) (width 1) (layer "B.Cu") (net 4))
 (segment (start 80.01 38.06) (end 80.01 50.6) (width 1) (layer "B.Cu") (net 4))
 (segment (start 83.815 54.405) (end 83.815 68.575) (width 1) (layer "B.Cu") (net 4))
 (segment (start 145.27 128.76) (end 145.27 130.81) (width 1) (layer "B.Cu") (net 18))
 (segment (start 99.06 114.3) (end 130.81 114.3) (width 1) (layer "B.Cu") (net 18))
 (segment (start 130.81 114.3) (end 145.27 128.76) (width 1) (layer "B.Cu") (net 18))
 (segment (start 83.815 83.815) (end 83.815 99.055) (width 1) (layer "B.Cu") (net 18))
 (segment (start 83.815 99.055) (end 99.06 114.3) (width 1) (layer "B.Cu") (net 18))
 (segment (start 87.63 53.34) (end 90.17 50.8) (width 1) (layer "B.Cu") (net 2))
 (segment (start 90.17 50.8) (end 90.17 38.1) (width 1) (layer "B.Cu") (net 2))
 (segment (start 86.36 54.61) (end 86.355 54.61) (width 1) (layer "B.Cu") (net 2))
 (segment (start 87.63 53.34) (end 86.36 54.61) (width 1) (layer "B.Cu") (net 2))
 (segment (start 86.355 54.61) (end 86.355 68.575) (width 1) (layer "B.Cu") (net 2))
 (segment (start 68.575 109.215) (end 77.47 118.11) (width 1) (layer "B.Cu") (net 13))
 (segment (start 125.73 118.11) (end 132.57 124.95) (width 1) (layer "B.Cu") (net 13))
 (segment (start 77.47 118.11) (end 125.73 118.11) (width 1) (layer "B.Cu") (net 13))
 (segment (start 68.575 83.815) (end 68.575 109.215) (width 1) (layer "B.Cu") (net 13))
 (segment (start 132.57 124.95) (end 132.57 130.81) (width 1) (layer "B.Cu") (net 13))
 (segment (start 116.835 68.575) (end 116.845 68.575) (width 1) (layer "B.Cu") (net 34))
 (segment (start 116.845 68.575) (end 127 58.42) (width 1) (layer "B.Cu") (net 34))
 (segment (start 60.96 71.12) (end 60.96 109.22) (width 1) (layer "B.Cu") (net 11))
 (segment (start 60.96 109.22) (end 74.93 123.19) (width 1) (layer "B.Cu") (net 11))
 (segment (start 71.115 66.035) (end 69.85 64.77) (width 1) (layer "B.Cu") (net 11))
 (segment (start 71.115 68.575) (end 71.115 66.035) (width 1) (layer "B.Cu") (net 11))
 (segment (start 74.93 123.19) (end 123.19 123.19) (width 1) (layer "B.Cu") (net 11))
 (segment (start 69.85 64.77) (end 67.31 64.77) (width 1) (layer "B.Cu") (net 11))
 (segment (start 127.49 127.49) (end 127.49 130.81) (width 1) (layer "B.Cu") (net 11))
 (segment (start 67.31 64.77) (end 60.96 71.12) (width 1) (layer "B.Cu") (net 11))
 (segment (start 123.19 123.19) (end 127.49 127.49) (width 1) (layer "B.Cu") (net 11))
 (segment (start 165.735 81.915) (end 165.735 97.155) (width 1) (layer "B.Cu") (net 9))
 (segment (start 117.33 130.81) (end 117.33 127.805) (width 1) (layer "B.Cu") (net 9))
 (segment (start 165.735 64.135) (end 165.735 81.915) (width 1) (layer "B.Cu") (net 9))
 (segment (start 143.51 109.22) (end 156.63 109.22) (width 1) (layer "B.Cu") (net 9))
 (segment (start 40.64 76.2) (end 41.658233 76.2) (width 1) (layer "B.Cu") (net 9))
 (segment (start 91.435 68.575) (end 91.435 71.115) (width 1) (layer "B.Cu") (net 9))
 (segment (start 159.46 60.67) (end 165.735 66.945) (width 1) (layer "B.Cu") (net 9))
 (segment (start 165.735 57.785) (end 165.735 64.135) (width 1) (layer "B.Cu") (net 9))
 (segment (start 156.21 48.26) (end 165.735 57.785) (width 1) (layer "B.Cu") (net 9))
 (segment (start 117.33 127.805) (end 118.135 127) (width 1) (layer "B.Cu") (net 9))
 (segment (start 111.936956 33.02) (end 127 48.083044) (width 1) (layer "B.Cu") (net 9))
 (segment (start 156.63 109.22) (end 159.46 106.39) (width 1) (layer "B.Cu") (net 9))
 (segment (start 91.435 71.115) (end 96.515 76.195) (width 1) (layer "B.Cu") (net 9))
 (segment (start 40.64 41.91) (end 46.99 35.56) (width 1) (layer "B.Cu") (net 9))
 (segment (start 105.41 101.6) (end 135.89 101.6) (width 1) (layer "B.Cu") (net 9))
 (segment (start 96.515 83.815) (end 96.515 92.705) (width 1) (layer "B.Cu") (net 9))
 (segment (start 165.465 81.915) (end 165.735 81.915) (width 1) (layer "B.Cu") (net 9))
 (segment (start 73.66 33.02) (end 71.12 35.56) (width 1) (layer "B.Cu") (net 9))
 (segment (start 111.76 33.02) (end 111.936956 33.02) (width 1) (layer "B.Cu") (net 9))
 (segment (start 46.99 106.68) (end 77.557315 137.247315) (width 1) (layer "B.Cu") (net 9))
 (segment (start 135.89 101.6) (end 143.51 109.22) (width 1) (layer "B.Cu") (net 9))
 (segment (start 118.135 127) (end 121.92 127) (width 1) (layer "B.Cu") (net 9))
 (segment (start 127 48.083044) (end 127 48.26) (width 1) (layer "B.Cu") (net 9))
 (segment (start 46.99 81.531767) (end 46.99 106.68) (width 1) (layer "B.Cu") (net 9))
 (segment (start 159.46 91.15) (end 165.465 97.155) (width 1) (layer "B.Cu") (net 9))
 (segment (start 165.735 100.115) (end 159.46 106.39) (width 1) (layer "B.Cu") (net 9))
 (segment (start 73.66 33.02) (end 111.76 33.02) (width 1) (layer "B.Cu") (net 9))
 (segment (start 77.557315 137.247315) (end 120.827382 137.247315) (width 1) (layer "B.Cu") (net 9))
 (segment (start 40.64 76.2) (end 40.64 41.91) (width 1) (layer "B.Cu") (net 9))
 (segment (start 122.41 127.49) (end 122.41 130.81) (width 1) (layer "B.Cu") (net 9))
 (segment (start 121.92 127) (end 122.41 127.49) (width 1) (layer "B.Cu") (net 9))
 (segment (start 96.515 92.705) (end 105.41 101.6) (width 1) (layer "B.Cu") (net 9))
 (segment (start 165.735 97.155) (end 165.735 100.115) (width 1) (layer "B.Cu") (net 9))
 (segment (start 96.515 76.195) (end 96.515 83.815) (width 1) (layer "B.Cu") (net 9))
 (segment (start 71.12 35.56) (end 49.53 35.56) (width 1) (layer "B.Cu") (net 9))
 (segment (start 127 48.26) (end 156.21 48.26) (width 1) (layer "B.Cu") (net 9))
 (segment (start 120.827382 137.247315) (end 122.41 135.664697) (width 1) (layer "B.Cu") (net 9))
 (segment (start 41.658233 76.2) (end 46.99 81.531767) (width 1) (layer "B.Cu") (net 9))
 (segment (start 46.99 35.56) (end 49.53 35.56) (width 1) (layer "B.Cu") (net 9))
 (segment (start 159.46 75.91) (end 165.465 81.915) (width 1) (layer "B.Cu") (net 9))
 (segment (start 122.41 135.664697) (end 122.41 130.81) (width 1) (layer "B.Cu") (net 9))
 (segment (start 124.95 137.145904) (end 124.95 130.81) (width 1) (layer "B.Cu") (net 10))
 (segment (start 43.18 107.95) (end 74.93 139.7) (width 1) (layer "B.Cu") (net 10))
 (segment (start 122.395904 139.7) (end 124.95 137.145904) (width 1) (layer "B.Cu") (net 10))
 (segment (start 43.18 81.28) (end 43.18 107.95) (width 1) (layer "B.Cu") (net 10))
 (segment (start 74.93 139.7) (end 122.395904 139.7) (width 1) (layer "B.Cu") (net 10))
 (segment (start 114.79 130.81) (end 114.79 134.475) (width 1) (layer "B.Cu") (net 1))
 (segment (start 88.895 68.575) (end 88.895 76.195) (width 1) (layer "B.Cu") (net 1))
 (segment (start 154.94 53.34) (end 111.76 53.34) (width 1) (layer "B.Cu") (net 1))
 (segment (start 50.8 105.41) (end 80.01 134.62) (width 1) (layer "B.Cu") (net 1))
 (segment (start 80.01 35.56) (end 90.13 35.56) (width 1) (layer "B.Cu") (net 1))
 (segment (start 88.895 68.575) (end 88.895 58.425) (width 1) (layer "B.Cu") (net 1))
 (segment (start 156.21 54.61) (end 154.94 53.34) (width 1) (layer "B.Cu") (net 1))
 (segment (start 48.26 38.1) (end 49.53 38.1) (width 1) (layer "B.Cu") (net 1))
 (segment (start 90.13 35.56) (end 90.17 35.6) (width 1) (layer "B.Cu") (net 1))
 (segment (start 114.935 134.62) (end 118.11 134.62) (width 1) (layer "B.Cu") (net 1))
 (segment (start 88.895 76.195) (end 93.975 81.275) (width 1) (layer "B.Cu") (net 1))
 (segment (start 140.97 64.77) (end 149.86 64.77) (width 1) (layer "B.Cu") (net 1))
 (segment (start 93.98 35.6) (end 93.98 53.34) (width 1) (layer "B.Cu") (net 1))
 (segment (start 111.76 53.34) (end 93.98 53.34) (width 1) (layer "B.Cu") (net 1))
 (segment (start 93.975 81.275) (end 93.975 83.815) (width 1) (layer "B.Cu") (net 1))
 (segment (start 49.53 38.1) (end 72.39 38.1) (width 1) (layer "B.Cu") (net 1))
 (segment (start 155.575 69.215) (end 156.21 69.85) (width 1) (layer "B.Cu") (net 1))
 (segment (start 156.21 78.74) (end 144.78 78.74) (width 1) (layer "B.Cu") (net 1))
 (segment (start 88.895 58.425) (end 93.98 53.34) (width 1) (layer "B.Cu") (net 1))
 (segment (start 45.72 40.64) (end 48.26 38.1) (width 1) (layer "B.Cu") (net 1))
 (segment (start 118.11 134.62) (end 119.87 132.86) (width 1) (layer "B.Cu") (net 1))
 (segment (start 45.72 76.2) (end 50.8 81.28) (width 1) (layer "B.Cu") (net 1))
 (segment (start 153.67 95.25) (end 140.97 95.25) (width 1) (layer "B.Cu") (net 1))
 (segment (start 140.97 85.09) (end 140.97 95.25) (width 1) (layer "B.Cu") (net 1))
 (segment (start 45.72 76.2) (end 45.72 40.64) (width 1) (layer "B.Cu") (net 1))
 (segment (start 156.21 69.85) (end 156.21 54.61) (width 1) (layer "B.Cu") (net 1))
 (segment (start 156.21 69.85) (end 156.21 92.71) (width 1) (layer "B.Cu") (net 1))
 (segment (start 151.13 64.77) (end 155.575 69.215) (width 1) (layer "B.Cu") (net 1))
 (segment (start 74.93 35.56) (end 80.01 35.56) (width 1) (layer "B.Cu") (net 1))
 (segment (start 149.86 64.77) (end 151.13 64.77) (width 1) (layer "B.Cu") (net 1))
 (segment (start 144.78 78.74) (end 140.97 74.93) (width 1) (layer "B.Cu") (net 1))
 (segment (start 111.76 36.52) (end 111.76 53.34) (width 1) (layer "B.Cu") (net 1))
 (segment (start 119.87 132.86) (end 119.87 130.81) (width 1) (layer "B.Cu") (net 1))
 (segment (start 93.98 35.6) (end 90.17 35.6) (width 1) (layer "B.Cu") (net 1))
 (segment (start 72.39 38.1) (end 74.93 35.56) (width 1) (layer "B.Cu") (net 1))
 (segment (start 50.8 81.28) (end 50.8 105.41) (width 1) (layer "B.Cu") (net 1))
 (segment (start 80.01 134.62) (end 114.935 134.62) (width 1) (layer "B.Cu") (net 1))
 (segment (start 114.79 134.475) (end 114.935 134.62) (width 1) (layer "B.Cu") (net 1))
 (segment (start 156.21 92.71) (end 153.67 95.25) (width 1) (layer "B.Cu") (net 1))
 (segment (start 76.195 68.575) (end 76.195 66.035) (width 1) (layer "B.Cu") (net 28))
 (segment (start 76.195 66.035) (end 55.88 45.72) (width 1) (layer "B.Cu") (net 28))
 (segment (start 55.88 45.72) (end 49.53 45.72) (width 1) (layer "B.Cu") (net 28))
 (segment (start 49.53 40.64) (end 58.42 40.64) (width 1) (layer "B.Cu") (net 26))
 (segment (start 58.42 40.64) (end 81.275 63.495) (width 1) (layer "B.Cu") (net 26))
 (segment (start 81.275 63.495) (end 81.275 68.575) (width 1) (layer "B.Cu") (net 26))
 (segment (start 57.15 43.18) (end 78.735 64.765) (width 1) (layer "B.Cu") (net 27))
 (segment (start 78.735 64.765) (end 78.735 68.575) (width 1) (layer "B.Cu") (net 27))
 (segment (start 54.61 43.18) (end 57.15 43.18) (width 1) (layer "B.Cu") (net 27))
 (segment (start 49.53 43.18) (end 54.61 43.18) (width 1) (layer "B.Cu") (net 27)))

